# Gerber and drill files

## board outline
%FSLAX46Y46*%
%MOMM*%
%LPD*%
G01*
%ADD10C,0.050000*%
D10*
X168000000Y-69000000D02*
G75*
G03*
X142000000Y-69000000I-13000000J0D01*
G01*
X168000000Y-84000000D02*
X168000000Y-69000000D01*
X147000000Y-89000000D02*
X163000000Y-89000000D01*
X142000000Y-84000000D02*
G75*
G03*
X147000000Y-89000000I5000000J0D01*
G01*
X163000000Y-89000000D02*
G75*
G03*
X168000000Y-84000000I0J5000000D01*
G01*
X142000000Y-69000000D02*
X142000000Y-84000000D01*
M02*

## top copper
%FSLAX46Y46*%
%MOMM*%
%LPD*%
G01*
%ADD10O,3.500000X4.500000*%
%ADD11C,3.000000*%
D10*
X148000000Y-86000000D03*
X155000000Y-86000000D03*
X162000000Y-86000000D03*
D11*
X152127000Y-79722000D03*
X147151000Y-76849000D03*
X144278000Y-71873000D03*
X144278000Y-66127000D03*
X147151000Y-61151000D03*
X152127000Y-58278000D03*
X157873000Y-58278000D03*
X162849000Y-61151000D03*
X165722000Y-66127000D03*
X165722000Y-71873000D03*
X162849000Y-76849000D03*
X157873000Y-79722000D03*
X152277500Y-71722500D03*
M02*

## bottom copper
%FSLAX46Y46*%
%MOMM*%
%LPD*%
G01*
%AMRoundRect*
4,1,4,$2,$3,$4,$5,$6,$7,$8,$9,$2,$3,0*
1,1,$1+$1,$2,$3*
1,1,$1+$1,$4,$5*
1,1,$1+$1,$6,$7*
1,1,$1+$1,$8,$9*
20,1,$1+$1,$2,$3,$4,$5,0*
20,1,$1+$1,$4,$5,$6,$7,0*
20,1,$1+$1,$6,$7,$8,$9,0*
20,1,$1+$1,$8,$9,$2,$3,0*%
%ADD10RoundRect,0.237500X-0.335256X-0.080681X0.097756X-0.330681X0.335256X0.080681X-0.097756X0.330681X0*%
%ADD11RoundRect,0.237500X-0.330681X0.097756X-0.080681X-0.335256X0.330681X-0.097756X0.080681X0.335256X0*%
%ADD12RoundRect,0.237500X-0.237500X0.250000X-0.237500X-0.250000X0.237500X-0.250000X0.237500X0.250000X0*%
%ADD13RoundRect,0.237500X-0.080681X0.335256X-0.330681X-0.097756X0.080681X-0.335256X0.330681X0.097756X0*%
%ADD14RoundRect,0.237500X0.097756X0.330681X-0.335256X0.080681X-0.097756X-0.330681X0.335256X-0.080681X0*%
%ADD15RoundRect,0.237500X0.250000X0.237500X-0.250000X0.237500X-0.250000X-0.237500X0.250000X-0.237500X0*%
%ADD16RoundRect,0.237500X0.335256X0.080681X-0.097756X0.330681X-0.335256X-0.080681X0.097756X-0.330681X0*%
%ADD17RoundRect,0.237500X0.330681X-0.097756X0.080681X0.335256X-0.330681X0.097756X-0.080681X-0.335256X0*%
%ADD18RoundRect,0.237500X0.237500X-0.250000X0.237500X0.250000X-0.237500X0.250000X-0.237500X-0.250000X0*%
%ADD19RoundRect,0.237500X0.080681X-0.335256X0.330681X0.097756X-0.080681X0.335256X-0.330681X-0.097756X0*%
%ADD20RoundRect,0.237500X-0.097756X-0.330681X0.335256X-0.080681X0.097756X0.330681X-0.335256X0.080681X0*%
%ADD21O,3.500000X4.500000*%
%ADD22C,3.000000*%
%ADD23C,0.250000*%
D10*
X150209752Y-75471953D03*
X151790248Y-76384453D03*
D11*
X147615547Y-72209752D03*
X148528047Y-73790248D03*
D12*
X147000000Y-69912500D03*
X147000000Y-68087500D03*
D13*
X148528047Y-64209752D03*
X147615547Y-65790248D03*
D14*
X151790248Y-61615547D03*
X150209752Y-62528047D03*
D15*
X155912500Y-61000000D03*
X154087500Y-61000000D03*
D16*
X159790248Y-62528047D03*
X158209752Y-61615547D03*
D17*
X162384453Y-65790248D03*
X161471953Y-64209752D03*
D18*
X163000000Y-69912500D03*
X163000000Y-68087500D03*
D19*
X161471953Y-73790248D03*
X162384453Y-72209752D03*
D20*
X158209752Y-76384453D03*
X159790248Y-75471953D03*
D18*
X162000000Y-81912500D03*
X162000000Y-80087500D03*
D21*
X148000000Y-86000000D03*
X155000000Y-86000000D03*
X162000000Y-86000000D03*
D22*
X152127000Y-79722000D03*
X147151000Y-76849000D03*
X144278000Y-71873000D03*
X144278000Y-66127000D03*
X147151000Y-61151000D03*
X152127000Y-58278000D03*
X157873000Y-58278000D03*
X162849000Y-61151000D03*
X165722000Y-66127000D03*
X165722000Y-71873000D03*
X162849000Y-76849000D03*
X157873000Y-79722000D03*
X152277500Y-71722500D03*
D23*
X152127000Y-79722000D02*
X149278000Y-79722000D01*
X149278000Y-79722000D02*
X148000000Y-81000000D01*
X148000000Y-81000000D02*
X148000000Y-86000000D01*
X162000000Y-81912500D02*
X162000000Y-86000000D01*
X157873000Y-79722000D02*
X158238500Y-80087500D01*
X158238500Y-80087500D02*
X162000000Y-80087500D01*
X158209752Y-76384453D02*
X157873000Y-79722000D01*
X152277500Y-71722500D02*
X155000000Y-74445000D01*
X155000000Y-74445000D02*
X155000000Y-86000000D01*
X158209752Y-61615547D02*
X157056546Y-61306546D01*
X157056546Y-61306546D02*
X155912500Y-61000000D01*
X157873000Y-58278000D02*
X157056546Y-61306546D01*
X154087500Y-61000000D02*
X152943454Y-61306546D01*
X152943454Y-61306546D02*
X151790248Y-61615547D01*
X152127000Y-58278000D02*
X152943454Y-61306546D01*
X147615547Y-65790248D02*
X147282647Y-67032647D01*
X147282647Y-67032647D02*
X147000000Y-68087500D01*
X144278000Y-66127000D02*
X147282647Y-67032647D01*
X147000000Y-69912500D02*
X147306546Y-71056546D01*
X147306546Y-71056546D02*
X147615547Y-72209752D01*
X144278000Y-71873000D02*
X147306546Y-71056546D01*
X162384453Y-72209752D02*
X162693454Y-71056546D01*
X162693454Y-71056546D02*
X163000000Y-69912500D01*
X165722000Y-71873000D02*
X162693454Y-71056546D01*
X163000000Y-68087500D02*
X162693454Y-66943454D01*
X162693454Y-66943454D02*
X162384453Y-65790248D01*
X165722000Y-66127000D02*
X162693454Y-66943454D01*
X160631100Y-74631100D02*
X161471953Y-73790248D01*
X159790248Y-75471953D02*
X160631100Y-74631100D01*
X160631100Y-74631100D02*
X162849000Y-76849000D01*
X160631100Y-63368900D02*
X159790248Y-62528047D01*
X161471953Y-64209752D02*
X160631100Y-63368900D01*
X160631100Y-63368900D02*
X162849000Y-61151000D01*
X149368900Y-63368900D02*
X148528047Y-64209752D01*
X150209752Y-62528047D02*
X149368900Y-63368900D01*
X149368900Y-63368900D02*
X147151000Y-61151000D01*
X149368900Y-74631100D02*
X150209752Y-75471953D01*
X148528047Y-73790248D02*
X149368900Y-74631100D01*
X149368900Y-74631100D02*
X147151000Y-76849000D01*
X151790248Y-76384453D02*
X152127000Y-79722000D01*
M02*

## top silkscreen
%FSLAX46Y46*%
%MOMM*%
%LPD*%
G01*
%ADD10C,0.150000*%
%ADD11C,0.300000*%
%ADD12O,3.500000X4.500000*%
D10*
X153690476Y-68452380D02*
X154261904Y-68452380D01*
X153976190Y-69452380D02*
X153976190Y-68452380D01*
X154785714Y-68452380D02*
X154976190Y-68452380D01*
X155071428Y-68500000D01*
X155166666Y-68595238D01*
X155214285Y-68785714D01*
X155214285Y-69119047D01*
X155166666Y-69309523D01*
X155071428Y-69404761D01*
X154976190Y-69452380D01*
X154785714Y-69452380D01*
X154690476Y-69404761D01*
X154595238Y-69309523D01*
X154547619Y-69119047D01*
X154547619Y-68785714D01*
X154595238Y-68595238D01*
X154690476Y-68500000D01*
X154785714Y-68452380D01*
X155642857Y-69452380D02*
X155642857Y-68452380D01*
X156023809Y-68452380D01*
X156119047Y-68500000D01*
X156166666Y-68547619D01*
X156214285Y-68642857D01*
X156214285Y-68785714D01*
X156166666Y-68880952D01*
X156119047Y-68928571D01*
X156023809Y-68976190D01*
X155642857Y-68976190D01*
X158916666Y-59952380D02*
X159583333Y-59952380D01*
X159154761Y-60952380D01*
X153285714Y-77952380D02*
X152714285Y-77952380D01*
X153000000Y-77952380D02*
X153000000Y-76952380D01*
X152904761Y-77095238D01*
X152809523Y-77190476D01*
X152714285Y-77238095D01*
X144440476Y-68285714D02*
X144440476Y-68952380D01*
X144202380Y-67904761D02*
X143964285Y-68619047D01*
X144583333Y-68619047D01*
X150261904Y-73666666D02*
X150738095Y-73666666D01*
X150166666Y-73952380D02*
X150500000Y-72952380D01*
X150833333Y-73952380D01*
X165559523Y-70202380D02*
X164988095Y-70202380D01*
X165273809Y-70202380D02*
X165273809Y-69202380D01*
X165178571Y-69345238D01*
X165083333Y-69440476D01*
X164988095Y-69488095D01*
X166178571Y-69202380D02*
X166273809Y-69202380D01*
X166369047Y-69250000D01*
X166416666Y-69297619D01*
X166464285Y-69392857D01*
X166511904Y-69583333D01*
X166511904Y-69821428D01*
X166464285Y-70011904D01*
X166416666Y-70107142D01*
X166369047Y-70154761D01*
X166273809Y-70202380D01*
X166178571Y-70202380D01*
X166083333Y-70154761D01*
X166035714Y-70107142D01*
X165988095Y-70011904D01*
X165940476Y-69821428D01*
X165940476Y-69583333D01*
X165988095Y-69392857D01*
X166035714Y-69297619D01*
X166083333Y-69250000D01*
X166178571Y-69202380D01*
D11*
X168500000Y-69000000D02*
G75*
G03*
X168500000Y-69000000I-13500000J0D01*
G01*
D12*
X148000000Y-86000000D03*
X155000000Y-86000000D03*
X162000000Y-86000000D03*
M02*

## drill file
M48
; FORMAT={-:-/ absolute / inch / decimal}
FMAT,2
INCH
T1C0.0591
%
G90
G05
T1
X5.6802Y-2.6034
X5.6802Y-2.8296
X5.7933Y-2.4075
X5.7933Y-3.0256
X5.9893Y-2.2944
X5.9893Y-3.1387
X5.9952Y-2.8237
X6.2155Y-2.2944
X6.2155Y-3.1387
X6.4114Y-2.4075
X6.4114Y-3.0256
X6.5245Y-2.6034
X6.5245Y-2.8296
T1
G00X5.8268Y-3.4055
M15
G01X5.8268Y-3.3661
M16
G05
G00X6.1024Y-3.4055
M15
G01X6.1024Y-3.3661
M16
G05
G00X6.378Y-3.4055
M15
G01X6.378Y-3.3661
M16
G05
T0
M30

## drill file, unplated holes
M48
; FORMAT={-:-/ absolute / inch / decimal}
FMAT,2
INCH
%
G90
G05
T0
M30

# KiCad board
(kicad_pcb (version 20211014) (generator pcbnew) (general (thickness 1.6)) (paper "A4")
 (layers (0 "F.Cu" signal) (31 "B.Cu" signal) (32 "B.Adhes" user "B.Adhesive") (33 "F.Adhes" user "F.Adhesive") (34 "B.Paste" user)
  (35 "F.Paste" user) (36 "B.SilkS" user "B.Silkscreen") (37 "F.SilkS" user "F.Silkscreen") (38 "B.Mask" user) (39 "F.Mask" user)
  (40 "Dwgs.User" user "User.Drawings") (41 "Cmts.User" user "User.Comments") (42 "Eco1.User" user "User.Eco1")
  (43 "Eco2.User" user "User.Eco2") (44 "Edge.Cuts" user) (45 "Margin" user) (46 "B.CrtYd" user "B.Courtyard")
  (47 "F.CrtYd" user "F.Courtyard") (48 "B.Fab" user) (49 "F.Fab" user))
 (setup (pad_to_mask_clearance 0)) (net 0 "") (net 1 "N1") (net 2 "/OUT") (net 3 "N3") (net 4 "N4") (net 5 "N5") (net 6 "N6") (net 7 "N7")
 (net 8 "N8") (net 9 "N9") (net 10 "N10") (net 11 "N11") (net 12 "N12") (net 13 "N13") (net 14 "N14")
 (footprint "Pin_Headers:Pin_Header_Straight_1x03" (layer "F.Cu") (at 155 86 90)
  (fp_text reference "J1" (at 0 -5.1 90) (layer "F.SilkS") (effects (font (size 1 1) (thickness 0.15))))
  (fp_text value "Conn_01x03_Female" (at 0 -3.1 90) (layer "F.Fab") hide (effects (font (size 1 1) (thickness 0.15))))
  (pad "1" thru_hole oval locked (at 0 -7 90) (size 4.5 3.5) (drill oval 2.5 1.5) (layers *.Cu *.Mask "F.SilkS") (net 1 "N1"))
  (pad "2" thru_hole oval locked (at 0 0 90) (size 4.5 3.5) (drill oval 2.5 1.5) (layers *.Cu *.Mask "F.SilkS") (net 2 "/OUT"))
  (pad "3" thru_hole oval locked (at 0 7 90) (size 4.5 3.5) (drill oval 2.5 1.5) (layers *.Cu *.Mask "F.SilkS") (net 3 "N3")))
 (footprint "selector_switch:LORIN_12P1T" (layer "F.Cu") (at 155 69)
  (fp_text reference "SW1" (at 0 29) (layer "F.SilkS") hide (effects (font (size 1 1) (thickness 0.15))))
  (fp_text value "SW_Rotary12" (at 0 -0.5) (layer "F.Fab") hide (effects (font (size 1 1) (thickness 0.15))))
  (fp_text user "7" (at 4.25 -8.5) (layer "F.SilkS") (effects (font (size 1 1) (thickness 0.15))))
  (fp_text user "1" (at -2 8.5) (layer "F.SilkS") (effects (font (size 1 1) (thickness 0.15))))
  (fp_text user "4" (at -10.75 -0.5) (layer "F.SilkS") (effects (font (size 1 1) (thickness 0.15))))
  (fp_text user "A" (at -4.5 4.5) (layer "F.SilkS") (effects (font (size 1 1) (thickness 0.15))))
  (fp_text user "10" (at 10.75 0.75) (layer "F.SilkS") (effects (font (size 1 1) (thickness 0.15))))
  (fp_circle (center 0 0) (end 13.5 0) (layer "F.SilkS") (width 0.3) (fill none))
  (pad "1" thru_hole circle locked (at -2.873 10.722 270) (size 3 3) (drill 1.5) (layers *.Cu *.Mask) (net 1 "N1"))
  (pad "2" thru_hole circle locked (at -7.849 7.849 270) (size 3 3) (drill 1.5) (layers *.Cu *.Mask) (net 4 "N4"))
  (pad "3" thru_hole circle locked (at -10.722 2.873 270) (size 3 3) (drill 1.5) (layers *.Cu *.Mask) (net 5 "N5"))
  (pad "4" thru_hole circle locked (at -10.722 -2.873 180) (size 3 3) (drill 1.5) (layers *.Cu *.Mask) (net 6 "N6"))
  (pad "5" thru_hole circle locked (at -7.849 -7.849 180) (size 3 3) (drill 1.5) (layers *.Cu *.Mask) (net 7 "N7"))
  (pad "6" thru_hole circle locked (at -2.873 -10.722 180) (size 3 3) (drill 1.5) (layers *.Cu *.Mask) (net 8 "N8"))
  (pad "7" thru_hole circle locked (at 2.873 -10.722 90) (size 3 3) (drill 1.5) (layers *.Cu *.Mask) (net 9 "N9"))
  (pad "8" thru_hole circle locked (at 7.849 -7.849 90) (size 3 3) (drill 1.5) (layers *.Cu *.Mask) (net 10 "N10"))
  (pad "9" thru_hole circle locked (at 10.722 -2.873 90) (size 3 3) (drill 1.5) (layers *.Cu *.Mask) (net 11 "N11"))
  (pad "10" thru_hole circle locked (at 10.722 2.873) (size 3 3) (drill 1.5) (layers *.Cu *.Mask) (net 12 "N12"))
  (pad "11" thru_hole circle locked (at 7.849 7.849) (size 3 3) (drill 1.5) (layers *.Cu *.Mask) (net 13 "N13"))
  (pad "12" thru_hole circle locked (at 2.873 10.722) (size 3 3) (drill 1.5) (layers *.Cu *.Mask) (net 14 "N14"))
  (pad "13" thru_hole circle locked (at -2.7225 2.7225 270) (size 3 3) (drill 1.5) (layers *.Cu *.Mask) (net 2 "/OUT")))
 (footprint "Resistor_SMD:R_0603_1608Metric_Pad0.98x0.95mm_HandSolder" (layer "B.Cu") (at 159 75.928203 30)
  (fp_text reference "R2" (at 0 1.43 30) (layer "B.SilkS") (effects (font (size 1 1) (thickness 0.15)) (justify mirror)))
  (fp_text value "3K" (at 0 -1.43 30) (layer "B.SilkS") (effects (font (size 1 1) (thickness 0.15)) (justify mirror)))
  (pad "1" smd roundrect (at -0.9125 0 30) (size 0.975 0.95) (layers "B.Cu" "B.Paste" "B.Mask") (roundrect_rratio 0.25) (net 14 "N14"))
  (pad "2" smd roundrect (at 0.9125 0 30) (size 0.975 0.95) (layers "B.Cu" "B.Paste" "B.Mask") (roundrect_rratio 0.25) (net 13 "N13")))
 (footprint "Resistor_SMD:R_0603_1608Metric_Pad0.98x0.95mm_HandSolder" (layer "B.Cu") (at 161.928203 65 120)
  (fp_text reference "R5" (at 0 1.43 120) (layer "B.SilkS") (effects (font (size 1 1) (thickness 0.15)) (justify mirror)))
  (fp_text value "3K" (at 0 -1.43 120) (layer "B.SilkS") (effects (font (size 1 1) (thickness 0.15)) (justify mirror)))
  (pad "1" smd roundrect (at -0.9125 0 120) (size 0.975 0.95) (layers "B.Cu" "B.Paste" "B.Mask") (roundrect_rratio 0.25) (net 11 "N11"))
  (pad "2" smd roundrect (at 0.9125 0 120) (size 0.975 0.95) (layers "B.Cu" "B.Paste" "B.Mask") (roundrect_rratio 0.25) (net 10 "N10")))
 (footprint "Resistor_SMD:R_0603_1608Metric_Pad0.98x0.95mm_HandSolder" (layer "B.Cu") (at 159 62.071797 150)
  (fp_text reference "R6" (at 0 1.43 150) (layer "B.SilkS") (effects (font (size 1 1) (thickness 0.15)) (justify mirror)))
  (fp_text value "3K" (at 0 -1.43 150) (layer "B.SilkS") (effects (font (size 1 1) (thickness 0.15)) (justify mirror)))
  (pad "1" smd roundrect (at -0.9125 0 150) (size 0.975 0.95) (layers "B.Cu" "B.Paste" "B.Mask") (roundrect_rratio 0.25) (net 10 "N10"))
  (pad "2" smd roundrect (at 0.9125 0 150) (size 0.975 0.95) (layers "B.Cu" "B.Paste" "B.Mask") (roundrect_rratio 0.25) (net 9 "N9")))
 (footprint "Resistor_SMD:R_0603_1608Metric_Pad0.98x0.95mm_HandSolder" (layer "B.Cu") (at 147 69 -90)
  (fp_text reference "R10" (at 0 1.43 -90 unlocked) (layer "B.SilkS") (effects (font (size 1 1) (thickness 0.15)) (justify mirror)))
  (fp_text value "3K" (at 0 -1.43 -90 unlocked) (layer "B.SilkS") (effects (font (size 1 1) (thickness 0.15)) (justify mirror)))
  (pad "1" smd roundrect (at -0.9125 0 270) (size 0.975 0.95) (layers "B.Cu" "B.Paste" "B.Mask") (roundrect_rratio 0.25) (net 6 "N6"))
  (pad "2" smd roundrect (at 0.9125 0 270) (size 0.975 0.95) (layers "B.Cu" "B.Paste" "B.Mask") (roundrect_rratio 0.25) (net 5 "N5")))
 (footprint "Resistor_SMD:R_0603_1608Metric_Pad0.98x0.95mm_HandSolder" (layer "B.Cu") (at 161.928203 73 60)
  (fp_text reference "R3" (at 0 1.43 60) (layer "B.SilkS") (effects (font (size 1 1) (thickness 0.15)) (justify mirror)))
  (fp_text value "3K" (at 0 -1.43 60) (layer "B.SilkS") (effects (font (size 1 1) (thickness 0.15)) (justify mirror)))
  (pad "1" smd roundrect (at -0.9125 0 60) (size 0.975 0.95) (layers "B.Cu" "B.Paste" "B.Mask") (roundrect_rratio 0.25) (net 13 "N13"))
  (pad "2" smd roundrect (at 0.9125 0 60) (size 0.975 0.95) (layers "B.Cu" "B.Paste" "B.Mask") (roundrect_rratio 0.25) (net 12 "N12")))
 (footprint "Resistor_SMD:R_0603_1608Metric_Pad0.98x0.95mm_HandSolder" (layer "B.Cu") (at 148.071797 65 -120)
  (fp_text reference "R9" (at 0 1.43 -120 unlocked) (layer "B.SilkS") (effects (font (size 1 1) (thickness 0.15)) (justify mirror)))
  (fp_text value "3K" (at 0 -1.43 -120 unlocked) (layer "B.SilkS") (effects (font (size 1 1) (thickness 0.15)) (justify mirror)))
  (pad "1" smd roundrect (at -0.9125 0 240) (size 0.975 0.95) (layers "B.Cu" "B.Paste" "B.Mask") (roundrect_rratio 0.25) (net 7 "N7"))
  (pad "2" smd roundrect (at 0.9125 0 240) (size 0.975 0.95) (layers "B.Cu" "B.Paste" "B.Mask") (roundrect_rratio 0.25) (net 6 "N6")))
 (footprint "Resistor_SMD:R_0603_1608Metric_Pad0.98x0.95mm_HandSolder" (layer "B.Cu") (at 155 61 180)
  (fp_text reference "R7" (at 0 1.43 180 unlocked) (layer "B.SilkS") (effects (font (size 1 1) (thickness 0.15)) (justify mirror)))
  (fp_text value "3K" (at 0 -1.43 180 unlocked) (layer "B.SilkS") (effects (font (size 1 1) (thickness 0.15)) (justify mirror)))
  (pad "1" smd roundrect (at -0.9125 0 180) (size 0.975 0.95) (layers "B.Cu" "B.Paste" "B.Mask") (roundrect_rratio 0.25) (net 9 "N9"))
  (pad "2" smd roundrect (at 0.9125 0 180) (size 0.975 0.95) (layers "B.Cu" "B.Paste" "B.Mask") (roundrect_rratio 0.25) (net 8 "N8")))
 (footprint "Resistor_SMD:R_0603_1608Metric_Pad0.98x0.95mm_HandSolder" (layer "B.Cu") (at 162 81 90)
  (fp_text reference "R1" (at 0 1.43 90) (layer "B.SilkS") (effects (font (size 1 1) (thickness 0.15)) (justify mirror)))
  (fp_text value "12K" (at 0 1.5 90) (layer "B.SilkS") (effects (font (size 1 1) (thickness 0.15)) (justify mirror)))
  (pad "1" smd roundrect (at -0.9125 0 90) (size 0.975 0.95) (layers "B.Cu" "B.Paste" "B.Mask") (roundrect_rratio 0.25) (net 3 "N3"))
  (pad "2" smd roundrect (at 0.9125 0 90) (size 0.975 0.95) (layers "B.Cu" "B.Paste" "B.Mask") (roundrect_rratio 0.25) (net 14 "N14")))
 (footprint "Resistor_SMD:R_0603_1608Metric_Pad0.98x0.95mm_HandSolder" (layer "B.Cu") (at 163 69 90)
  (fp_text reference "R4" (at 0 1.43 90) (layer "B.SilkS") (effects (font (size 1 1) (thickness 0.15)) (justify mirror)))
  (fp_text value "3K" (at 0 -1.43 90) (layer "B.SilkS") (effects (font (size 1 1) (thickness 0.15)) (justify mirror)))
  (pad "1" smd roundrect (at -0.9125 0 90) (size 0.975 0.95) (layers "B.Cu" "B.Paste" "B.Mask") (roundrect_rratio 0.25) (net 12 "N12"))
  (pad "2" smd roundrect (at 0.9125 0 90) (size 0.975 0.95) (layers "B.Cu" "B.Paste" "B.Mask") (roundrect_rratio 0.25) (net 11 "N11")))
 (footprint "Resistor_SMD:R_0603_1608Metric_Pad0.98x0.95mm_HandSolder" (layer "B.Cu") (at 151 62.071797 -150)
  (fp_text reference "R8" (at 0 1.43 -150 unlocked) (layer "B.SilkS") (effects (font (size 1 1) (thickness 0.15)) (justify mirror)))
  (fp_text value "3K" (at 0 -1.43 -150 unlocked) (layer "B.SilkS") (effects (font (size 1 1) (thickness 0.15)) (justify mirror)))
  (pad "1" smd roundrect (at -0.9125 0 210) (size 0.975 0.95) (layers "B.Cu" "B.Paste" "B.Mask") (roundrect_rratio 0.25) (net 8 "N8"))
  (pad "2" smd roundrect (at 0.9125 0 210) (size 0.975 0.95) (layers "B.Cu" "B.Paste" "B.Mask") (roundrect_rratio 0.25) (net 7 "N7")))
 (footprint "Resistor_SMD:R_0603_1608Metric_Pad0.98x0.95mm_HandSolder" (layer "B.Cu") (at 151 75.928203 -30)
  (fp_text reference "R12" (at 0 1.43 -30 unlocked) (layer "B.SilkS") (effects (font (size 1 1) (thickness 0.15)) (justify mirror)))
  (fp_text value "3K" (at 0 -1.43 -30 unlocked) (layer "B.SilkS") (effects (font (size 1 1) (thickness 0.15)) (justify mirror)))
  (pad "1" smd roundrect (at -0.9125 0 330) (size 0.975 0.95) (layers "B.Cu" "B.Paste" "B.Mask") (roundrect_rratio 0.25) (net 4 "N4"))
  (pad "2" smd roundrect (at 0.9125 0 330) (size 0.975 0.95) (layers "B.Cu" "B.Paste" "B.Mask") (roundrect_rratio 0.25) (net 1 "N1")))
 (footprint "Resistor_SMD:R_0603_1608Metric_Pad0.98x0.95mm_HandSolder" (layer "B.Cu") (at 148.071797 73 -60)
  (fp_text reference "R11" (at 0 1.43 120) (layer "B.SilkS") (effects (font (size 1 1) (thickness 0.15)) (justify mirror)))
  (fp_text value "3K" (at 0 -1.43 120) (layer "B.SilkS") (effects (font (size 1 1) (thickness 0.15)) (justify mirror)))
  (pad "1" smd roundrect (at -0.9125 0 300) (size 0.975 0.95) (layers "B.Cu" "B.Paste" "B.Mask") (roundrect_rratio 0.25) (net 5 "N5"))
  (pad "2" smd roundrect (at 0.9125 0 300) (size 0.975 0.95) (layers "B.Cu" "B.Paste" "B.Mask") (roundrect_rratio 0.25) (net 4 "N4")))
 (gr_arc (start 142 69) (mid 155 56) (end 168 69) (layer "Edge.Cuts") (width 0.05))
 (gr_line (start 168 84) (end 168 69) (layer "Edge.Cuts") (width 0.05))
 (gr_line (start 147 89) (end 163 89) (layer "Edge.Cuts") (width 0.05))
 (gr_arc (start 147 89) (mid 143.464466 87.535534) (end 142 84) (layer "Edge.Cuts") (width 0.05))
 (gr_arc (start 168 84) (mid 166.535534 87.535534) (end 163 89) (layer "Edge.Cuts") (width 0.05))
 (gr_line (start 142 69) (end 142 84) (layer "Edge.Cuts") (width 0.05))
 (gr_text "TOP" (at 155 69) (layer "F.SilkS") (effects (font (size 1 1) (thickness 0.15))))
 (segment (start 152.2775 71.7225) (end 155 74.445) (width 0.25) (layer "B.Cu") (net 2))
 (segment (start 155 74.445) (end 155 86) (width 0.25) (layer "B.Cu") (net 2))
 (segment (start 152.127 79.722) (end 149.278 79.722) (width 0.25) (layer "B.Cu") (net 1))
 (segment (start 148 81) (end 148 86) (width 0.25) (layer "B.Cu") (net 1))
 (segment (start 151.790248 76.384453) (end 152.127 79.722) (width 0.25) (layer "B.Cu") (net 1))
 (segment (start 149.278 79.722) (end 148 81) (width 0.25) (layer "B.Cu") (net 1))
 (segment (start 162 81.9125) (end 162 86) (width 0.25) (layer "B.Cu") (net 3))
 (segment (start 159.790248 75.471953) (end 160.6311 74.6311) (width 0.25) (layer "B.Cu") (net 13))
 (segment (start 160.6311 74.6311) (end 161.471953 73.790248) (width 0.25) (layer "B.Cu") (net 13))
 (segment (start 160.6311 74.6311) (end 162.849 76.849) (width 0.25) (layer "B.Cu") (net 13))
 (segment (start 162.384453 72.209752) (end 162.693454 71.056546) (width 0.25) (layer "B.Cu") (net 12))
 (segment (start 162.693454 71.056546) (end 163 69.9125) (width 0.25) (layer "B.Cu") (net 12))
 (segment (start 165.722 71.873) (end 162.693454 71.056546) (width 0.25) (layer "B.Cu") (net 12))
 (segment (start 165.722 66.127) (end 162.693454 66.943454) (width 0.25) (layer "B.Cu") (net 11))
 (segment (start 162.693454 66.943454) (end 162.384453 65.790248) (width 0.25) (layer "B.Cu") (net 11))
 (segment (start 163 68.0875) (end 162.693454 66.943454) (width 0.25) (layer "B.Cu") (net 11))
 (segment (start 160.6311 63.3689) (end 162.849 61.151) (width 0.25) (layer "B.Cu") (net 10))
 (segment (start 160.6311 63.3689) (end 159.790248 62.528047) (width 0.25) (layer "B.Cu") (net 10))
 (segment (start 161.471953 64.209752) (end 160.6311 63.3689) (width 0.25) (layer "B.Cu") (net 10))
 (segment (start 157.056546 61.306546) (end 155.9125 61) (width 0.25) (layer "B.Cu") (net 9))
 (segment (start 157.873 58.278) (end 157.056546 61.306546) (width 0.25) (layer "B.Cu") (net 9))
 (segment (start 158.209752 61.615547) (end 157.056546 61.306546) (width 0.25) (layer "B.Cu") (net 9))
 (segment (start 144.278 66.127) (end 147.282647 67.032647) (width 0.25) (layer "B.Cu") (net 6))
 (segment (start 147.615547 65.790248) (end 147.282647 67.032647) (width 0.25) (layer "B.Cu") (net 6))
 (segment (start 147.282647 67.032647) (end 147 68.0875) (width 0.25) (layer "B.Cu") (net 6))
 (segment (start 149.3689 63.3689) (end 148.528047 64.209752) (width 0.25) (layer "B.Cu") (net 7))
 (segment (start 149.3689 63.3689) (end 147.151 61.151) (width 0.25) (layer "B.Cu") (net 7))
 (segment (start 150.209752 62.528047) (end 149.3689 63.3689) (width 0.25) (layer "B.Cu") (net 7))
 (segment (start 158.209752 76.384453) (end 157.873 79.722) (width 0.25) (layer "B.Cu") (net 14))
 (segment (start 157.873 79.722) (end 158.2385 80.0875) (width 0.25) (layer "B.Cu") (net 14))
 (segment (start 158.2385 80.0875) (end 162 80.0875) (width 0.25) (layer "B.Cu") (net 14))
 (segment (start 147.306546 71.056546) (end 147.615547 72.209752) (width 0.25) (layer "B.Cu") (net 5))
 (segment (start 144.278 71.873) (end 147.306546 71.056546) (width 0.25) (layer "B.Cu") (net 5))
 (segment (start 147 69.9125) (end 147.306546 71.056546) (width 0.25) (layer "B.Cu") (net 5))
 (segment (start 148.528047 73.790248) (end 149.3689 74.6311) (width 0.25) (layer "B.Cu") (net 4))
 (segment (start 149.3689 74.6311) (end 147.151 76.849) (width 0.25) (layer "B.Cu") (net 4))
 (segment (start 149.3689 74.6311) (end 150.209752 75.471953) (width 0.25) (layer "B.Cu") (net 4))
 (segment (start 152.943454 61.306546) (end 151.790248 61.615547) (width 0.25) (layer "B.Cu") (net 8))
 (segment (start 152.127 58.278) (end 152.943454 61.306546) (width 0.25) (layer "B.Cu") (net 8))
 (segment (start 154.0875 61) (end 152.943454 61.306546) (width 0.25) (layer "B.Cu") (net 8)))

